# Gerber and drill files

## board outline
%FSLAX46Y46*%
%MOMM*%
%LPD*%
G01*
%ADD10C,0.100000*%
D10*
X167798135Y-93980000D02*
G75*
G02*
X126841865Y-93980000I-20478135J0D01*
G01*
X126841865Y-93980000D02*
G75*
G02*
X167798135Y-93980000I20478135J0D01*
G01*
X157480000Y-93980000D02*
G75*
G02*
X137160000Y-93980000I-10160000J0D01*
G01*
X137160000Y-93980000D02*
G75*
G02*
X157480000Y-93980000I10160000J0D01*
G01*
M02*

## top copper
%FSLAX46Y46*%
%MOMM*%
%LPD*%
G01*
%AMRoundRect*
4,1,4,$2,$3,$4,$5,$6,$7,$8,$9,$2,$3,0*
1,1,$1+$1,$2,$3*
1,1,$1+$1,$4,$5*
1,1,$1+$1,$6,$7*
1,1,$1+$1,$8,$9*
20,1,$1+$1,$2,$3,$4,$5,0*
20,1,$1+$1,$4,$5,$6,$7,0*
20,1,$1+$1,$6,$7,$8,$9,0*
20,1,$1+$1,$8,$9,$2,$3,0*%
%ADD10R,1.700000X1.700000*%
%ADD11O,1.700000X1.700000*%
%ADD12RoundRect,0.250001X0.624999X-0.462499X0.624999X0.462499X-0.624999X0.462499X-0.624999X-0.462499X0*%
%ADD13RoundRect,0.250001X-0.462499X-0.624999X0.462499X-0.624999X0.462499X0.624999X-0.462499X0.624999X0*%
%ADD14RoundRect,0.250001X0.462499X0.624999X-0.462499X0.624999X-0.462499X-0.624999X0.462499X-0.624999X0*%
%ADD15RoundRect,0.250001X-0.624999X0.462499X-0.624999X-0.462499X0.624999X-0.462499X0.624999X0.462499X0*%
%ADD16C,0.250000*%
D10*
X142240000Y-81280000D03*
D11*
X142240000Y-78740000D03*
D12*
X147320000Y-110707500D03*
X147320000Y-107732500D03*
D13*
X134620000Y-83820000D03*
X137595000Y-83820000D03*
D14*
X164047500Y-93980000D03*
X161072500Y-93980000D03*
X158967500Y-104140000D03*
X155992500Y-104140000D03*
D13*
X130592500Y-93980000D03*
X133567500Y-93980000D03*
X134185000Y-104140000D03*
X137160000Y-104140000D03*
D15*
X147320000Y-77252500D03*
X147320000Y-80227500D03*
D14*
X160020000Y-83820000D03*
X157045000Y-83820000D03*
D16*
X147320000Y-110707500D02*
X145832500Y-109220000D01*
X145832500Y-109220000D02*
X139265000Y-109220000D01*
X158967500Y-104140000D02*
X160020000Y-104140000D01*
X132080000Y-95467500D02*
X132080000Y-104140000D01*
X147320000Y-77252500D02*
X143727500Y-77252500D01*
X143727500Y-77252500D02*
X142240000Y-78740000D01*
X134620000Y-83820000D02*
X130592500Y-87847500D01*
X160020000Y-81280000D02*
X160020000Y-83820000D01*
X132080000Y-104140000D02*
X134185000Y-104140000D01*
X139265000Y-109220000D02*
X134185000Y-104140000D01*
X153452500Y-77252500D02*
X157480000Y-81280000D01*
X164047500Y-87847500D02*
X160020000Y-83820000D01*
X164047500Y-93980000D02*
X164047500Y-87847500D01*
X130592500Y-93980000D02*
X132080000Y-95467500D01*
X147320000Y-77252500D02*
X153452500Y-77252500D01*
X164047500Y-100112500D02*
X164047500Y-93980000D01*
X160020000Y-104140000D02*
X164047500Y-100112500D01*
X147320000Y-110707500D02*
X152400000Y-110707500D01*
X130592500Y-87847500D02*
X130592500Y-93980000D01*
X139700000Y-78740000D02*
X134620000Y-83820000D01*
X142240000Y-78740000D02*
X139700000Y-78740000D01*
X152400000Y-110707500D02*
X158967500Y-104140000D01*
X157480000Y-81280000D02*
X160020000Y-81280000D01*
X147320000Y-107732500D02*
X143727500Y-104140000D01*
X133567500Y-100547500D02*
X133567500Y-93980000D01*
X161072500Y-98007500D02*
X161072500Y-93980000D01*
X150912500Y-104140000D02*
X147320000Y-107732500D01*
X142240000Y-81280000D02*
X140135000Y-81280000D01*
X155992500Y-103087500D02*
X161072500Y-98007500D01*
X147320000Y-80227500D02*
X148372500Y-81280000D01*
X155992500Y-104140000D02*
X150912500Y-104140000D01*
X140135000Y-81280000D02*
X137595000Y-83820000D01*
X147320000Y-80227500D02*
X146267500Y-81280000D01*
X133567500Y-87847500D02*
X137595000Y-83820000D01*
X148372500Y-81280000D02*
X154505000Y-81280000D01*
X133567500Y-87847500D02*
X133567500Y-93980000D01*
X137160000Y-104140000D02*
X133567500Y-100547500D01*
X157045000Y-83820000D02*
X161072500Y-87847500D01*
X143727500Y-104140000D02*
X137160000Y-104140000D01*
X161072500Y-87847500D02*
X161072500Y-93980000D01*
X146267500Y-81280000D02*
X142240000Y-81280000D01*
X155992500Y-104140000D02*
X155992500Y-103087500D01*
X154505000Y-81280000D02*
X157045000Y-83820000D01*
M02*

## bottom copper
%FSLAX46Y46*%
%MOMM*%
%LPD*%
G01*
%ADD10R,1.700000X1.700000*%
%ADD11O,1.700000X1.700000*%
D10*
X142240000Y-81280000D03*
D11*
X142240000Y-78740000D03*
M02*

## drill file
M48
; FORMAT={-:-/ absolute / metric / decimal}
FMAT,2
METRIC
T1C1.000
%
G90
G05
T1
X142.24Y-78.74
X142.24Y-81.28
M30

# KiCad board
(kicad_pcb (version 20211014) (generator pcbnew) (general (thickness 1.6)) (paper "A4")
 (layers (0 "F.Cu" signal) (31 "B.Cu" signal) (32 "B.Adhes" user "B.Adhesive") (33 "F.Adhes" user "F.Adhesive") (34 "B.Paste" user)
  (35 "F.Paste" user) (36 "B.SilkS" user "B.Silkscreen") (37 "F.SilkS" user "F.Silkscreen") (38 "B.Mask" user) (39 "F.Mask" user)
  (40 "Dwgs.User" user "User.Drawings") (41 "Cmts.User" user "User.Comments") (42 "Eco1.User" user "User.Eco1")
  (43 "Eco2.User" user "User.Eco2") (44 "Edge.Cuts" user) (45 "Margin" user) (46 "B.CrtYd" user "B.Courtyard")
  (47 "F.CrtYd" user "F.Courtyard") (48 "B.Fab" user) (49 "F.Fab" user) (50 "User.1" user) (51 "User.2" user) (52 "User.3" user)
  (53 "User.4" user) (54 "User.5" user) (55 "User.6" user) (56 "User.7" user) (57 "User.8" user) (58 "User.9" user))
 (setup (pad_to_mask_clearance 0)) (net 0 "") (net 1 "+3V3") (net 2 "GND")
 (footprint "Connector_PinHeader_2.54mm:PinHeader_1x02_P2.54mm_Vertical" (layer "F.Cu") (at 142.24 81.28 180)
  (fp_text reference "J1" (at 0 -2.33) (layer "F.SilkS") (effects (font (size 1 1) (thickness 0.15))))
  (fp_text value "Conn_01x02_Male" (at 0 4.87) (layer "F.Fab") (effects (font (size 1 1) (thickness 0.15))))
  (pad "1" thru_hole rect (at 0 0 180) (size 1.7 1.7) (drill 1) (layers *.Cu *.Mask) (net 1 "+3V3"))
  (pad "2" thru_hole oval (at 0 2.54 180) (size 1.7 1.7) (drill 1) (layers *.Cu *.Mask) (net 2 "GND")))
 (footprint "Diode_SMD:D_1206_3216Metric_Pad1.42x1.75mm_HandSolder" (layer "F.Cu") (at 147.32 109.22 90)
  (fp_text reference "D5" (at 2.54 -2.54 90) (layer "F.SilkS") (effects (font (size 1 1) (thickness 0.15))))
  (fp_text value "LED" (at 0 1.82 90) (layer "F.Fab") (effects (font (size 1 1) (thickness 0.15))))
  (pad "1" smd roundrect (at -1.4875 0 90) (size 1.425 1.75) (layers "F.Cu" "F.Paste" "F.Mask") (roundrect_rratio 0.175439) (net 2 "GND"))
  (pad "2" smd roundrect (at 1.4875 0 90) (size 1.425 1.75) (layers "F.Cu" "F.Paste" "F.Mask") (roundrect_rratio 0.175439) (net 1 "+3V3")))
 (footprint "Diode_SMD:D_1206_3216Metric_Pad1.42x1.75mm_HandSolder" (layer "F.Cu") (at 136.1075 83.82)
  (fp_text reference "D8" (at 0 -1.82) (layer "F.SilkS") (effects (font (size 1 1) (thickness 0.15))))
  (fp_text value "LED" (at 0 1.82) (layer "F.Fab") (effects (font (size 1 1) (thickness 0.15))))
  (pad "1" smd roundrect (at -1.4875 0) (size 1.425 1.75) (layers "F.Cu" "F.Paste" "F.Mask") (roundrect_rratio 0.175439) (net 2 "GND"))
  (pad "2" smd roundrect (at 1.4875 0) (size 1.425 1.75) (layers "F.Cu" "F.Paste" "F.Mask") (roundrect_rratio 0.175439) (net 1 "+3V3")))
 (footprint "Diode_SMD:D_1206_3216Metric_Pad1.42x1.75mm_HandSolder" (layer "F.Cu") (at 162.56 93.98 180)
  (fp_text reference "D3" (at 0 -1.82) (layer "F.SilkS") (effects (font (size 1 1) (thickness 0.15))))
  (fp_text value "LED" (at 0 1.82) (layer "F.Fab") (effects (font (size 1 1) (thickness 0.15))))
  (pad "1" smd roundrect (at -1.4875 0 180) (size 1.425 1.75) (layers "F.Cu" "F.Paste" "F.Mask") (roundrect_rratio 0.175439) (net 2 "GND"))
  (pad "2" smd roundrect (at 1.4875 0 180) (size 1.425 1.75) (layers "F.Cu" "F.Paste" "F.Mask") (roundrect_rratio 0.175439) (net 1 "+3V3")))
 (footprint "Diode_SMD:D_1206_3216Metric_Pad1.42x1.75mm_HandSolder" (layer "F.Cu") (at 157.48 104.14 180)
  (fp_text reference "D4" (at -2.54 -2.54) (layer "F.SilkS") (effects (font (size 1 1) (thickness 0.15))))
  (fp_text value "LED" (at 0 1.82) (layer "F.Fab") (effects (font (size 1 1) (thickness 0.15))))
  (pad "1" smd roundrect (at -1.4875 0 180) (size 1.425 1.75) (layers "F.Cu" "F.Paste" "F.Mask") (roundrect_rratio 0.175439) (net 2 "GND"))
  (pad "2" smd roundrect (at 1.4875 0 180) (size 1.425 1.75) (layers "F.Cu" "F.Paste" "F.Mask") (roundrect_rratio 0.175439) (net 1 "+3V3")))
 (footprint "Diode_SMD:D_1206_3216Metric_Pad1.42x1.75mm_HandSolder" (layer "F.Cu") (at 132.08 93.98)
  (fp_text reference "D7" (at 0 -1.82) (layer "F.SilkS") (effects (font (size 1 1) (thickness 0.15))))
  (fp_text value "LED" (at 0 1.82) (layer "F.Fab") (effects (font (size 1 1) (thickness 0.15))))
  (pad "1" smd roundrect (at -1.4875 0) (size 1.425 1.75) (layers "F.Cu" "F.Paste" "F.Mask") (roundrect_rratio 0.175439) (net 2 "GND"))
  (pad "2" smd roundrect (at 1.4875 0) (size 1.425 1.75) (layers "F.Cu" "F.Paste" "F.Mask") (roundrect_rratio 0.175439) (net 1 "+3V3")))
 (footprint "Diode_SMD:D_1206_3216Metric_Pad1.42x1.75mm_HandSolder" (layer "F.Cu") (at 135.6725 104.14)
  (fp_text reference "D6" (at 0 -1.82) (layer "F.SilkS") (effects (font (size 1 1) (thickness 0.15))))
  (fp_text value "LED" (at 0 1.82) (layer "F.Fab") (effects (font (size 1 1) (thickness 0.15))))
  (pad "1" smd roundrect (at -1.4875 0) (size 1.425 1.75) (layers "F.Cu" "F.Paste" "F.Mask") (roundrect_rratio 0.175439) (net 2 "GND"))
  (pad "2" smd roundrect (at 1.4875 0) (size 1.425 1.75) (layers "F.Cu" "F.Paste" "F.Mask") (roundrect_rratio 0.175439) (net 1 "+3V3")))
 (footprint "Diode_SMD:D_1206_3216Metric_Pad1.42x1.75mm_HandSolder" (layer "F.Cu") (at 147.32 78.74 -90)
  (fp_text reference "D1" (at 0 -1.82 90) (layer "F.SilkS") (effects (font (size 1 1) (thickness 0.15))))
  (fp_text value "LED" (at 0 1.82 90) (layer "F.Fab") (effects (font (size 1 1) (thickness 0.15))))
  (pad "1" smd roundrect (at -1.4875 0 270) (size 1.425 1.75) (layers "F.Cu" "F.Paste" "F.Mask") (roundrect_rratio 0.175439) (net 2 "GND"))
  (pad "2" smd roundrect (at 1.4875 0 270) (size 1.425 1.75) (layers "F.Cu" "F.Paste" "F.Mask") (roundrect_rratio 0.175439) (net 1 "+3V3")))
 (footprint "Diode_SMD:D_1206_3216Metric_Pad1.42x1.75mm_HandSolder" (layer "F.Cu") (at 158.5325 83.82 180)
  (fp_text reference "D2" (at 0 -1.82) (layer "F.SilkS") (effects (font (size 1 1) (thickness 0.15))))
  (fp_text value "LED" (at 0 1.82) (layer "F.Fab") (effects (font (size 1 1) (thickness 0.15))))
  (pad "1" smd roundrect (at -1.4875 0 180) (size 1.425 1.75) (layers "F.Cu" "F.Paste" "F.Mask") (roundrect_rratio 0.175439) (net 2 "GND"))
  (pad "2" smd roundrect (at 1.4875 0 180) (size 1.425 1.75) (layers "F.Cu" "F.Paste" "F.Mask") (roundrect_rratio 0.175439) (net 1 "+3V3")))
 (gr_circle (center 147.32 93.98) (end 167.64 91.44) (layer "Edge.Cuts") (width 0.1) (fill none))
 (gr_circle (center 147.32 93.98) (end 157.48 93.98) (layer "Edge.Cuts") (width 0.1) (fill none))
 (segment (start 147.32 110.7075) (end 145.8325 109.22) (width 0.25) (layer "F.Cu") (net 2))
 (segment (start 145.8325 109.22) (end 139.265 109.22) (width 0.25) (layer "F.Cu") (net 2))
 (segment (start 158.9675 104.14) (end 160.02 104.14) (width 0.25) (layer "F.Cu") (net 2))
 (segment (start 132.08 95.4675) (end 132.08 104.14) (width 0.25) (layer "F.Cu") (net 2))
 (segment (start 147.32 77.2525) (end 143.7275 77.2525) (width 0.25) (layer "F.Cu") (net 2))
 (segment (start 143.7275 77.2525) (end 142.24 78.74) (width 0.25) (layer "F.Cu") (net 2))
 (segment (start 134.62 83.82) (end 130.5925 87.8475) (width 0.25) (layer "F.Cu") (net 2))
 (segment (start 160.02 81.28) (end 160.02 83.82) (width 0.25) (layer "F.Cu") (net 2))
 (segment (start 132.08 104.14) (end 134.185 104.14) (width 0.25) (layer "F.Cu") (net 2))
 (segment (start 139.265 109.22) (end 134.185 104.14) (width 0.25) (layer "F.Cu") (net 2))
 (segment (start 153.4525 77.2525) (end 157.48 81.28) (width 0.25) (layer "F.Cu") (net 2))
 (segment (start 164.0475 87.8475) (end 160.02 83.82) (width 0.25) (layer "F.Cu") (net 2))
 (segment (start 164.0475 93.98) (end 164.0475 87.8475) (width 0.25) (layer "F.Cu") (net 2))
 (segment (start 130.5925 93.98) (end 132.08 95.4675) (width 0.25) (layer "F.Cu") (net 2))
 (segment (start 147.32 77.2525) (end 153.4525 77.2525) (width 0.25) (layer "F.Cu") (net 2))
 (segment (start 164.0475 100.1125) (end 164.0475 93.98) (width 0.25) (layer "F.Cu") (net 2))
 (segment (start 160.02 104.14) (end 164.0475 100.1125) (width 0.25) (layer "F.Cu") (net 2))
 (segment (start 147.32 110.7075) (end 152.4 110.7075) (width 0.25) (layer "F.Cu") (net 2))
 (segment (start 130.5925 87.8475) (end 130.5925 93.98) (width 0.25) (layer "F.Cu") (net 2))
 (segment (start 139.7 78.74) (end 134.62 83.82) (width 0.25) (layer "F.Cu") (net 2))
 (segment (start 142.24 78.74) (end 139.7 78.74) (width 0.25) (layer "F.Cu") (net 2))
 (segment (start 152.4 110.7075) (end 158.9675 104.14) (width 0.25) (layer "F.Cu") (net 2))
 (segment (start 157.48 81.28) (end 160.02 81.28) (width 0.25) (layer "F.Cu") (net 2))
 (segment (start 147.32 107.7325) (end 143.7275 104.14) (width 0.25) (layer "F.Cu") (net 1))
 (segment (start 133.5675 100.5475) (end 133.5675 93.98) (width 0.25) (layer "F.Cu") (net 1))
 (segment (start 161.0725 98.0075) (end 161.0725 93.98) (width 0.25) (layer "F.Cu") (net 1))
 (segment (start 150.9125 104.14) (end 147.32 107.7325) (width 0.25) (layer "F.Cu") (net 1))
 (segment (start 142.24 81.28) (end 140.135 81.28) (width 0.25) (layer "F.Cu") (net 1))
 (segment (start 155.9925 103.0875) (end 161.0725 98.0075) (width 0.25) (layer "F.Cu") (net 1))
 (segment (start 147.32 80.2275) (end 148.3725 81.28) (width 0.25) (layer "F.Cu") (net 1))
 (segment (start 155.9925 104.14) (end 150.9125 104.14) (width 0.25) (layer "F.Cu") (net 1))
 (segment (start 140.135 81.28) (end 137.595 83.82) (width 0.25) (layer "F.Cu") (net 1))
 (segment (start 147.32 80.2275) (end 146.2675 81.28) (width 0.25) (layer "F.Cu") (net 1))
 (segment (start 133.5675 87.8475) (end 137.595 83.82) (width 0.25) (layer "F.Cu") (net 1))
 (segment (start 148.3725 81.28) (end 154.505 81.28) (width 0.25) (layer "F.Cu") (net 1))
 (segment (start 133.5675 87.8475) (end 133.5675 93.98) (width 0.25) (layer "F.Cu") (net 1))
 (segment (start 137.16 104.14) (end 133.5675 100.5475) (width 0.25) (layer "F.Cu") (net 1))
 (segment (start 157.045 83.82) (end 161.0725 87.8475) (width 0.25) (layer "F.Cu") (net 1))
 (segment (start 143.7275 104.14) (end 137.16 104.14) (width 0.25) (layer "F.Cu") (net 1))
 (segment (start 161.0725 87.8475) (end 161.0725 93.98) (width 0.25) (layer "F.Cu") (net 1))
 (segment (start 146.2675 81.28) (end 142.24 81.28) (width 0.25) (layer "F.Cu") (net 1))
 (segment (start 155.9925 104.14) (end 155.9925 103.0875) (width 0.25) (layer "F.Cu") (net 1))
 (segment (start 154.505 81.28) (end 157.045 83.82) (width 0.25) (layer "F.Cu") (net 1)))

